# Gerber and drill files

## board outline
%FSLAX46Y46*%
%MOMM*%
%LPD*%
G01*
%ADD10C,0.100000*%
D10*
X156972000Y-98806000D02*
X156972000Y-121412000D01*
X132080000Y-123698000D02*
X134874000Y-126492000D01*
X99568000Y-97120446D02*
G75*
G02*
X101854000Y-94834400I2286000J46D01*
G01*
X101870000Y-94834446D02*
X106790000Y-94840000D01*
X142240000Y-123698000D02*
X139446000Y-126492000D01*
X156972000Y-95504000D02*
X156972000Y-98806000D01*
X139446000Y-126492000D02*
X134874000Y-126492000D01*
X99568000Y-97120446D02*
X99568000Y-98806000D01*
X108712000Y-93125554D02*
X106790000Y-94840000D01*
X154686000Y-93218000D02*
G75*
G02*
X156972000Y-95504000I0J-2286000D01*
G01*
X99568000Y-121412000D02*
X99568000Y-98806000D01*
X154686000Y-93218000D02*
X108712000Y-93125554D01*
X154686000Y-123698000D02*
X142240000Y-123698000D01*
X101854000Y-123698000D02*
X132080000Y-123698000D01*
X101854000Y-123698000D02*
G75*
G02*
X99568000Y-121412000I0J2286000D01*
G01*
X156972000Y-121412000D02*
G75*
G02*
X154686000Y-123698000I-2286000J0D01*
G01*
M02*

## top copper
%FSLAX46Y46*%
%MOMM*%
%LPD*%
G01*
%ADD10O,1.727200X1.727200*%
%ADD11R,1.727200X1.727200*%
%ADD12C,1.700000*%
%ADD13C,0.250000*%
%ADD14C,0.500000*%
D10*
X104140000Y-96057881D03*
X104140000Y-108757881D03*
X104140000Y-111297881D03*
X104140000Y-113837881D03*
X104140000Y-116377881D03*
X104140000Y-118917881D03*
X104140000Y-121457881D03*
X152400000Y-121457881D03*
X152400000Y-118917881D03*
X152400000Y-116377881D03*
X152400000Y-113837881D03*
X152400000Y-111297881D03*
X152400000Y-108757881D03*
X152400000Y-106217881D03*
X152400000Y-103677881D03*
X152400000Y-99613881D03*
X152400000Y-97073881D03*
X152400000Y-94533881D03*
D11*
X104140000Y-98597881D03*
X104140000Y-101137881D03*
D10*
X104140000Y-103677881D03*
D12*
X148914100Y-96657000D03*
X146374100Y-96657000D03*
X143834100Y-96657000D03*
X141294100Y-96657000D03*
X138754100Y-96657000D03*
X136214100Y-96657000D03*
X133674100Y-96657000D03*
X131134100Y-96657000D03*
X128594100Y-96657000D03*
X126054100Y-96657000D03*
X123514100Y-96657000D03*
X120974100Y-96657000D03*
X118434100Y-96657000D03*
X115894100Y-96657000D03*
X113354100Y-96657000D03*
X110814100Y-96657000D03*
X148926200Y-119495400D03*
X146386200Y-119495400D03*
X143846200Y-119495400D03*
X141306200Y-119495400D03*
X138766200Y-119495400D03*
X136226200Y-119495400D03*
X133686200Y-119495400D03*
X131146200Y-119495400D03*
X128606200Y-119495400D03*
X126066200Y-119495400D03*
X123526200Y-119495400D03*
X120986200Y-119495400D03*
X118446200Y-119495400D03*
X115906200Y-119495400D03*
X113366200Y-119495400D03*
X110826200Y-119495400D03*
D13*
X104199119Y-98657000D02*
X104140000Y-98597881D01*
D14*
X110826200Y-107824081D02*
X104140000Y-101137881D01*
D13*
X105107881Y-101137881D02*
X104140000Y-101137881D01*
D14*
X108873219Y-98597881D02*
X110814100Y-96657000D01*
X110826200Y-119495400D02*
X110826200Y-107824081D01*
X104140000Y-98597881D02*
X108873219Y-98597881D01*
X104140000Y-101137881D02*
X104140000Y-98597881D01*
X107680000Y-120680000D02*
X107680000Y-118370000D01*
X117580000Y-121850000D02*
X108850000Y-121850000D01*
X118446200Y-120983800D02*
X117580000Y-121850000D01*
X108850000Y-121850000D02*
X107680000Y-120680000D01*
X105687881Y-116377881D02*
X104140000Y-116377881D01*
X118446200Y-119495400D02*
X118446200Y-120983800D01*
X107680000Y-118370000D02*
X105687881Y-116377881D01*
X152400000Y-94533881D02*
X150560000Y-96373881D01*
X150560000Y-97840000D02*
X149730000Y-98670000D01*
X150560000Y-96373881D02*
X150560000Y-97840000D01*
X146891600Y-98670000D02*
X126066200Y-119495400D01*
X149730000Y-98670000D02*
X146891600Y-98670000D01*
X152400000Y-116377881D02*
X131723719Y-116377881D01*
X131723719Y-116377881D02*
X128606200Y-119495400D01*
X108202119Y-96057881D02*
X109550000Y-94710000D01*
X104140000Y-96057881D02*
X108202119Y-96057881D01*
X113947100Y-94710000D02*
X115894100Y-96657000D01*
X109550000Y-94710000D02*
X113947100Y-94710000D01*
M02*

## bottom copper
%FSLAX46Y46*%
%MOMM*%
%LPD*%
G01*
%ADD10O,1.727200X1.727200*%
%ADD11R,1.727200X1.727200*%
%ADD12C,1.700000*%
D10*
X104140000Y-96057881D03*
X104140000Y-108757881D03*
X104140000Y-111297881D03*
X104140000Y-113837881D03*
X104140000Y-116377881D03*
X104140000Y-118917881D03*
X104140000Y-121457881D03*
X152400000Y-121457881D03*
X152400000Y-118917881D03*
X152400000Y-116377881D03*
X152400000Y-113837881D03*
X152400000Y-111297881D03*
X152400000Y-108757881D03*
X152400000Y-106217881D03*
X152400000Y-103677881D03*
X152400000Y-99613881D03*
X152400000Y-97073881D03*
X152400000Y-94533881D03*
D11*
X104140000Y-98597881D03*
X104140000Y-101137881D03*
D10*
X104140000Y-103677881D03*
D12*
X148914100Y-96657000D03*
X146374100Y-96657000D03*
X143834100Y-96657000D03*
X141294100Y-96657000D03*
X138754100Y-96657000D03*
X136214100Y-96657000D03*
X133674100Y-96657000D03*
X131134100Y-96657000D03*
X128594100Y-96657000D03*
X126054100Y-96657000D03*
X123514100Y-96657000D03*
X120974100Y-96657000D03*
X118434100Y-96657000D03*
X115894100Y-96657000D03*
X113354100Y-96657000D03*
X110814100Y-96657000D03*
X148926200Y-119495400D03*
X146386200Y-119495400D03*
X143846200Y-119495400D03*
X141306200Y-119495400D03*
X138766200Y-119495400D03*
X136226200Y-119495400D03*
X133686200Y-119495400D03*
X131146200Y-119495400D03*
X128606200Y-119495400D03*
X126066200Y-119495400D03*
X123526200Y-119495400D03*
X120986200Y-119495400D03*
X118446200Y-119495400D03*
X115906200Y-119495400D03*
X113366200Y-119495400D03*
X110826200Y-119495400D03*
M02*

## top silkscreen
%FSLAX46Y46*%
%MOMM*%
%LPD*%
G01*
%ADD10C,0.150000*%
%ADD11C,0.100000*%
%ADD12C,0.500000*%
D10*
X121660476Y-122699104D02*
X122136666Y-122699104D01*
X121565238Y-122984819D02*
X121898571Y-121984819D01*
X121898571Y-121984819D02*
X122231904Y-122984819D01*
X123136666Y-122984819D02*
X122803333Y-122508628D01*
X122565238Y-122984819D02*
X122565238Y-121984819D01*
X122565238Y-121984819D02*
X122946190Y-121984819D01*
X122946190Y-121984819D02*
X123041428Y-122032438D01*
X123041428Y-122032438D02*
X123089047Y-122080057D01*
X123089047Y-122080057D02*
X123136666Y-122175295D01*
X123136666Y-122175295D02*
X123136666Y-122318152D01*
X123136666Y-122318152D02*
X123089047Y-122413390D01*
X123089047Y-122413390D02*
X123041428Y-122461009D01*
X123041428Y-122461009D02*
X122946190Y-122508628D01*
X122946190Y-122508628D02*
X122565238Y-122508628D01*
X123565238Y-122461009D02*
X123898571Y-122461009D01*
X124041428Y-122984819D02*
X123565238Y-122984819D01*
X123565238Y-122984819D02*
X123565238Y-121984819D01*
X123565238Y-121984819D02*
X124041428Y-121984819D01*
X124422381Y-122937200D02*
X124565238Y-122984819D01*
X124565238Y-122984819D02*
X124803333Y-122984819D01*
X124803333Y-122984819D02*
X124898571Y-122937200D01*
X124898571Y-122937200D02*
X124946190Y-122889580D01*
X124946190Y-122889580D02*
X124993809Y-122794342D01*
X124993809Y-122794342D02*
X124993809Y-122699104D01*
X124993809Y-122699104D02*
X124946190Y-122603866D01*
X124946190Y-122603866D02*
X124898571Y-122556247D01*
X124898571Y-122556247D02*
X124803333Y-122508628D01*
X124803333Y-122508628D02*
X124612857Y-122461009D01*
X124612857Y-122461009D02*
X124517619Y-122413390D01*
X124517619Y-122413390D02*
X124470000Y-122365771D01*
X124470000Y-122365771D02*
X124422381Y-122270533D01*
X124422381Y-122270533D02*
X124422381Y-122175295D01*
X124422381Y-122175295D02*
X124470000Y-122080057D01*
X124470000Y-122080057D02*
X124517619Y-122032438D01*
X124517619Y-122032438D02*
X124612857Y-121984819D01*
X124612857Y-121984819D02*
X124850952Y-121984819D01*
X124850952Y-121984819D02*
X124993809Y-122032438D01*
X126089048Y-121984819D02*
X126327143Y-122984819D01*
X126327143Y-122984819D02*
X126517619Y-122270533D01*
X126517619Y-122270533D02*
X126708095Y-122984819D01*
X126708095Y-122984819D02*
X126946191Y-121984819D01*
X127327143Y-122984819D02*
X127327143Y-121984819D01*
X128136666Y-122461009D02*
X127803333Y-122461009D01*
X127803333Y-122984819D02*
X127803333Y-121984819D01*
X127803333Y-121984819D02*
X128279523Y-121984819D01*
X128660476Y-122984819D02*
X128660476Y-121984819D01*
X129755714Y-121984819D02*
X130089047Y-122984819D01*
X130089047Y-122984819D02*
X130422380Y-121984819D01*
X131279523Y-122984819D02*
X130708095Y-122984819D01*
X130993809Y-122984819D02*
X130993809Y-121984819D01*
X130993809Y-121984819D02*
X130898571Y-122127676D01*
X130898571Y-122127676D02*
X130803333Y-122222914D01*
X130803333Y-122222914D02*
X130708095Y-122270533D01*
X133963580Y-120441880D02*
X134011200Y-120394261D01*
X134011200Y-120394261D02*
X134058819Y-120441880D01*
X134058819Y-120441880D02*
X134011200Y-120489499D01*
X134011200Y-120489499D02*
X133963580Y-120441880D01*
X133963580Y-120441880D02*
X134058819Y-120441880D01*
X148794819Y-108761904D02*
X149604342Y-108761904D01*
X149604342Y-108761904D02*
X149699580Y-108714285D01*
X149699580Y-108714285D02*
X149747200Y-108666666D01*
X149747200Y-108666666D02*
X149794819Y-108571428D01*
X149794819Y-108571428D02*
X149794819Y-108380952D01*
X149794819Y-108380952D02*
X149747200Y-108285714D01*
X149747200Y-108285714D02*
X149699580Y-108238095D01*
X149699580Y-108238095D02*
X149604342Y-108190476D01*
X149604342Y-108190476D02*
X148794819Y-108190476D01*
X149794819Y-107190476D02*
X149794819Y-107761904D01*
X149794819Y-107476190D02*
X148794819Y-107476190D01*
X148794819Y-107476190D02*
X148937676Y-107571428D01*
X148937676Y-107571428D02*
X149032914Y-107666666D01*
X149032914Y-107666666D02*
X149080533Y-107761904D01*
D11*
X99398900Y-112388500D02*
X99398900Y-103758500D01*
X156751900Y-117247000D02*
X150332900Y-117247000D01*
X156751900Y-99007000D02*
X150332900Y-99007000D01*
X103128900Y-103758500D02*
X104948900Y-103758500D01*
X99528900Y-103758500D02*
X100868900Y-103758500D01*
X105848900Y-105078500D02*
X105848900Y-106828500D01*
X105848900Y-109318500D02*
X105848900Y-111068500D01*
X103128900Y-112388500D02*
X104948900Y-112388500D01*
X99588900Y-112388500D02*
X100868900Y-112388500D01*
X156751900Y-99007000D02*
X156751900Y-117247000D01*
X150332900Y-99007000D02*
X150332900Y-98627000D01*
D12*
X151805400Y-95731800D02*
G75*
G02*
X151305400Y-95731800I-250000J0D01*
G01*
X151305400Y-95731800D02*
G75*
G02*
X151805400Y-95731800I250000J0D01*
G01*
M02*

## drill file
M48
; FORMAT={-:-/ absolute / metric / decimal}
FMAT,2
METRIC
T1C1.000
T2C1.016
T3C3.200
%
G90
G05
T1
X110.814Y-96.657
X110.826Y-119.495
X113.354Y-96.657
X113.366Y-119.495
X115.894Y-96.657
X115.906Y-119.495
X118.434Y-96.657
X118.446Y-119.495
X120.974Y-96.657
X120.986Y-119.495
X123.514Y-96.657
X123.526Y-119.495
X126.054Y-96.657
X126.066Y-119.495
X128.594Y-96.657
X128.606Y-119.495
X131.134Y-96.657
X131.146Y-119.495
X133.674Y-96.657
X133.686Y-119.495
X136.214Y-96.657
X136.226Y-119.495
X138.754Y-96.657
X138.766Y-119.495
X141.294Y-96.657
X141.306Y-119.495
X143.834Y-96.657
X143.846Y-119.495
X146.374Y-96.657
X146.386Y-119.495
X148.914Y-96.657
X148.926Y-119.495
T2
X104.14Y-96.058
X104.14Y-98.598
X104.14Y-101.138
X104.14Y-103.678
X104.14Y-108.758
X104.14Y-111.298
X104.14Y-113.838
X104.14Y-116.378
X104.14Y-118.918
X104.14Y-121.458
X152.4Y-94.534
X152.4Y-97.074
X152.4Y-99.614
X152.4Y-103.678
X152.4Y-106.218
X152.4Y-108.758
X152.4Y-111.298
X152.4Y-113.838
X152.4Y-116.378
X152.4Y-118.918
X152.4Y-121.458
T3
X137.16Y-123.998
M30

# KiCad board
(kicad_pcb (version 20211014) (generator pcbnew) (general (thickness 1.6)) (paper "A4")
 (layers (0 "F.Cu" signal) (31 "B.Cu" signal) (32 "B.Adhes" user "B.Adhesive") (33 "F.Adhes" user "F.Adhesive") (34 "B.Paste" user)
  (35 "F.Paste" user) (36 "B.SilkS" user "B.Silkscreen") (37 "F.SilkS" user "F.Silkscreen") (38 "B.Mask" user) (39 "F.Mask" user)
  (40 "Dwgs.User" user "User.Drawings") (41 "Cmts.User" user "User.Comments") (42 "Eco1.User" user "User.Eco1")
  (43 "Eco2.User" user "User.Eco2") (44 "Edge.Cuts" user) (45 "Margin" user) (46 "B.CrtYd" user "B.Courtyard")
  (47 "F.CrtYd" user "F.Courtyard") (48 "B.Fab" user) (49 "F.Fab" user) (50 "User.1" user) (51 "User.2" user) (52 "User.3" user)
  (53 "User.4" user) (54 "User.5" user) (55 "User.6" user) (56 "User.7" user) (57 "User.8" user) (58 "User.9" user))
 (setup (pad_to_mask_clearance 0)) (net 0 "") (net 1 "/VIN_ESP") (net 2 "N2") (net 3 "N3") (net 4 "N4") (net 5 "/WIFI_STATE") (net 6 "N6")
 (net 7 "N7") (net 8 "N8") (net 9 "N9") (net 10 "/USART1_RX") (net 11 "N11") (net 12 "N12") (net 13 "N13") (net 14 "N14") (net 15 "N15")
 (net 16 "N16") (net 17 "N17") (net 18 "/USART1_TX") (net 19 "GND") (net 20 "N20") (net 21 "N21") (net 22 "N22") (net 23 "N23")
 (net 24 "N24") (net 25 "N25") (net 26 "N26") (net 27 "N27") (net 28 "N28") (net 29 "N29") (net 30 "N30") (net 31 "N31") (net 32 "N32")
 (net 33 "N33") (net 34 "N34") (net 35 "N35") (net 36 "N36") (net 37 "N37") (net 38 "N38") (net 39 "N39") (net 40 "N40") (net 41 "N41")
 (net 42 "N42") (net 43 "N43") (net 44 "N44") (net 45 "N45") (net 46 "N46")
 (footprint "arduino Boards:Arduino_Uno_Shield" (layer "F.Cu") (at 101.6 57.957881 -90)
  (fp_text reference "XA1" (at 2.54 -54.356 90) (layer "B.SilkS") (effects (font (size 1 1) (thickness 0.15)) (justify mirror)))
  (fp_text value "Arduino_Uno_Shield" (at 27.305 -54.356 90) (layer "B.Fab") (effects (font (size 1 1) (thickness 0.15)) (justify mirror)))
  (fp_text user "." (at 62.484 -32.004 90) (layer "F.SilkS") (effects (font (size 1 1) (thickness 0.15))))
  (pad "" np_thru_hole circle (at 66.04 -35.56 270) (size 3.2 3.2) (drill 3.2) (layers *.Cu *.Mask))
  (pad "5V1" thru_hole oval (at 38.1 -2.54 270) (size 1.7272 1.7272) (drill 1.016) (layers *.Cu *.Mask) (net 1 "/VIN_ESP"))
  (pad "A0" thru_hole oval (at 50.8 -2.54 270) (size 1.7272 1.7272) (drill 1.016) (layers *.Cu *.Mask) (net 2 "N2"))
  (pad "A1" thru_hole oval (at 53.34 -2.54 270) (size 1.7272 1.7272) (drill 1.016) (layers *.Cu *.Mask) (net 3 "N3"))
  (pad "A2" thru_hole oval (at 55.88 -2.54 270) (size 1.7272 1.7272) (drill 1.016) (layers *.Cu *.Mask) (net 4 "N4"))
  (pad "A3" thru_hole oval (at 58.42 -2.54 270) (size 1.7272 1.7272) (drill 1.016) (layers *.Cu *.Mask) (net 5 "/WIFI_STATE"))
  (pad "A4" thru_hole oval (at 60.96 -2.54 270) (size 1.7272 1.7272) (drill 1.016) (layers *.Cu *.Mask) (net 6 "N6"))
  (pad "A5" thru_hole oval (at 63.5 -2.54 270) (size 1.7272 1.7272) (drill 1.016) (layers *.Cu *.Mask) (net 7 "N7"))
  (pad "D0" thru_hole oval (at 63.5 -50.8 270) (size 1.7272 1.7272) (drill 1.016) (layers *.Cu *.Mask) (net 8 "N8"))
  (pad "D1" thru_hole oval (at 60.96 -50.8 270) (size 1.7272 1.7272) (drill 1.016) (layers *.Cu *.Mask) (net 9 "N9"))
  (pad "D2" thru_hole oval (at 58.42 -50.8 270) (size 1.7272 1.7272) (drill 1.016) (layers *.Cu *.Mask) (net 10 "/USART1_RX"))
  (pad "D3" thru_hole oval (at 55.88 -50.8 270) (size 1.7272 1.7272) (drill 1.016) (layers *.Cu *.Mask) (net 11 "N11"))
  (pad "D4" thru_hole oval (at 53.34 -50.8 270) (size 1.7272 1.7272) (drill 1.016) (layers *.Cu *.Mask) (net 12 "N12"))
  (pad "D5" thru_hole oval (at 50.8 -50.8 270) (size 1.7272 1.7272) (drill 1.016) (layers *.Cu *.Mask) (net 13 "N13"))
  (pad "D6" thru_hole oval (at 48.26 -50.8 270) (size 1.7272 1.7272) (drill 1.016) (layers *.Cu *.Mask) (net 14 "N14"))
  (pad "D7" thru_hole oval (at 45.72 -50.8 270) (size 1.7272 1.7272) (drill 1.016) (layers *.Cu *.Mask) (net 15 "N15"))
  (pad "D8" thru_hole oval (at 41.656 -50.8 270) (size 1.7272 1.7272) (drill 1.016) (layers *.Cu *.Mask) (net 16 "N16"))
  (pad "D9" thru_hole oval (at 39.116 -50.8 270) (size 1.7272 1.7272) (drill 1.016) (layers *.Cu *.Mask) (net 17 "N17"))
  (pad "D10" thru_hole oval (at 36.576 -50.8 270) (size 1.7272 1.7272) (drill 1.016) (layers *.Cu *.Mask) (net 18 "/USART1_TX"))
  (pad "GND2" thru_hole rect (at 40.64 -2.54 270) (size 1.7272 1.7272) (drill 1.016) (layers *.Cu *.Mask) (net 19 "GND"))
  (pad "GND3" thru_hole rect (at 43.18 -2.54 270) (size 1.7272 1.7272) (drill 1.016) (layers *.Cu *.Mask) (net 19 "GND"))
  (pad "VIN" thru_hole oval (at 45.72 -2.54 270) (size 1.7272 1.7272) (drill 1.016) (layers *.Cu *.Mask) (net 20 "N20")))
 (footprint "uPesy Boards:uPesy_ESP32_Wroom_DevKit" (layer "F.Cu") (at 129.94 108 -90)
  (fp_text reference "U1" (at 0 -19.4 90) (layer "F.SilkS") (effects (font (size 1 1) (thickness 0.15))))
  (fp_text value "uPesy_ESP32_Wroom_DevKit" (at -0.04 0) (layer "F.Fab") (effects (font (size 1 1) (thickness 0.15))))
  (fp_line (start 4.3885 30.5411) (end -4.2415 30.5411) (layer "F.SilkS") (width 0.1))
  (fp_line (start 9.247 -26.8119) (end 9.247 -20.3929) (layer "F.SilkS") (width 0.1))
  (fp_line (start -8.993 -26.8119) (end -8.993 -20.3929) (layer "F.SilkS") (width 0.1))
  (fp_line (start -4.2415 26.8111) (end -4.2415 24.9911) (layer "F.SilkS") (width 0.1))
  (fp_line (start -4.2415 30.4111) (end -4.2415 29.0711) (layer "F.SilkS") (width 0.1))
  (fp_line (start -2.9215 24.0911) (end -1.1715 24.0911) (layer "F.SilkS") (width 0.1))
  (fp_line (start 1.3185 24.0911) (end 3.0685 24.0911) (layer "F.SilkS") (width 0.1))
  (fp_line (start 4.3885 26.8111) (end 4.3885 24.9911) (layer "F.SilkS") (width 0.1))
  (fp_line (start 4.3885 30.3511) (end 4.3885 29.0711) (layer "F.SilkS") (width 0.1))
  (fp_line (start -8.993 -26.8119) (end 9.247 -26.8119) (layer "F.SilkS") (width 0.1))
  (fp_line (start -8.993 -20.3929) (end -9.373 -20.3929) (layer "F.SilkS") (width 0.1))
  (fp_circle (center -12.2682 -21.6154) (end -12.0182 -21.6154) (layer "F.SilkS") (width 0.5) (fill none))
  (pad "1" thru_hole circle (at -11.343 -18.9741 180) (size 1.7 1.7) (drill 1) (layers *.Cu *.Mask) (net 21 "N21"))
  (pad "2" thru_hole circle (at -11.343 -16.4341 180) (size 1.7 1.7) (drill 1) (layers *.Cu *.Mask) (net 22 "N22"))
  (pad "3" thru_hole circle (at -11.343 -13.8941 180) (size 1.7 1.7) (drill 1) (layers *.Cu *.Mask) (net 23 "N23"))
  (pad "4" thru_hole circle (at -11.343 -11.3541 180) (size 1.7 1.7) (drill 1) (layers *.Cu *.Mask) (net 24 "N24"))
  (pad "5" thru_hole circle (at -11.343 -8.8141 180) (size 1.7 1.7) (drill 1) (layers *.Cu *.Mask) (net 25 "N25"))
  (pad "6" thru_hole circle (at -11.343 -6.2741 180) (size 1.7 1.7) (drill 1) (layers *.Cu *.Mask) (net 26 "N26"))
  (pad "7" thru_hole circle (at -11.343 -3.7341 180) (size 1.7 1.7) (drill 1) (layers *.Cu *.Mask) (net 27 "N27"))
  (pad "8" thru_hole circle (at -11.343 -1.1941 180) (size 1.7 1.7) (drill 1) (layers *.Cu *.Mask) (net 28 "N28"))
  (pad "9" thru_hole circle (at -11.343 1.3459 180) (size 1.7 1.7) (drill 1) (layers *.Cu *.Mask) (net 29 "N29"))
  (pad "10" thru_hole circle (at -11.343 3.8859 180) (size 1.7 1.7) (drill 1) (layers *.Cu *.Mask) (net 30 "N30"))
  (pad "11" thru_hole circle (at -11.343 6.4259 180) (size 1.7 1.7) (drill 1) (layers *.Cu *.Mask) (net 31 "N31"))
  (pad "12" thru_hole circle (at -11.343 8.9659 180) (size 1.7 1.7) (drill 1) (layers *.Cu *.Mask) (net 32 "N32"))
  (pad "13" thru_hole circle (at -11.343 11.5059 180) (size 1.7 1.7) (drill 1) (layers *.Cu *.Mask) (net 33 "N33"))
  (pad "14" thru_hole circle (at -11.343 14.0459 180) (size 1.7 1.7) (drill 1) (layers *.Cu *.Mask) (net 1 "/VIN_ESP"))
  (pad "15" thru_hole circle (at -11.343 16.5859 180) (size 1.7 1.7) (drill 1) (layers *.Cu *.Mask) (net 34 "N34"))
  (pad "16" thru_hole circle (at -11.343 19.1259 180) (size 1.7 1.7) (drill 1) (layers *.Cu *.Mask) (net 19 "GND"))
  (pad "17" thru_hole circle (at 11.4954 -18.9862) (size 1.7 1.7) (drill 1) (layers *.Cu *.Mask) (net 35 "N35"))
  (pad "18" thru_hole circle (at 11.4954 -16.4462) (size 1.7 1.7) (drill 1) (layers *.Cu *.Mask) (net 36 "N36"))
  (pad "19" thru_hole circle (at 11.4954 -13.9062) (size 1.7 1.7) (drill 1) (layers *.Cu *.Mask) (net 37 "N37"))
  (pad "20" thru_hole circle (at 11.4954 -11.3662) (size 1.7 1.7) (drill 1) (layers *.Cu *.Mask) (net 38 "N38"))
  (pad "21" thru_hole circle (at 11.4954 -8.8262) (size 1.7 1.7) (drill 1) (layers *.Cu *.Mask) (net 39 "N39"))
  (pad "22" thru_hole circle (at 11.4954 -6.2862) (size 1.7 1.7) (drill 1) (layers *.Cu *.Mask) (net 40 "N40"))
  (pad "23" thru_hole circle (at 11.4954 -3.7462) (size 1.7 1.7) (drill 1) (layers *.Cu *.Mask) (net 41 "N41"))
  (pad "24" thru_hole circle (at 11.4954 -1.2062) (size 1.7 1.7) (drill 1) (layers *.Cu *.Mask) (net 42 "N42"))
  (pad "25" thru_hole circle (at 11.4954 1.3338) (size 1.7 1.7) (drill 1) (layers *.Cu *.Mask) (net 10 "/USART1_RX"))
  (pad "26" thru_hole circle (at 11.4954 3.8738) (size 1.7 1.7) (drill 1) (layers *.Cu *.Mask) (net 18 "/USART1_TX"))
  (pad "27" thru_hole circle (at 11.4954 6.4138) (size 1.7 1.7) (drill 1) (layers *.Cu *.Mask) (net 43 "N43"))
  (pad "28" thru_hole circle (at 11.4954 8.9538) (size 1.7 1.7) (drill 1) (layers *.Cu *.Mask) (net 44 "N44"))
  (pad "29" thru_hole circle (at 11.4954 11.4938) (size 1.7 1.7) (drill 1) (layers *.Cu *.Mask) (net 5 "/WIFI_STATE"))
  (pad "30" thru_hole circle (at 11.4954 14.0338) (size 1.7 1.7) (drill 1) (layers *.Cu *.Mask) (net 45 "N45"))
  (pad "31" thru_hole circle (at 11.4954 16.5738) (size 1.7 1.7) (drill 1) (layers *.Cu *.Mask) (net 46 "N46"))
  (pad "32" thru_hole circle (at 11.4954 19.1138) (size 1.7 1.7) (drill 1) (layers *.Cu *.Mask) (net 19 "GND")))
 (gr_line (start 156.972 98.806) (end 156.972 121.412) (layer "Edge.Cuts") (width 0.1))
 (gr_line (start 132.08 123.698) (end 134.874 126.492) (layer "Edge.Cuts") (width 0.1))
 (gr_arc (start 99.568 97.120446) (mid 100.237554 95.504) (end 101.854 94.834446) (layer "Edge.Cuts") (width 0.1))
 (gr_line (start 101.87 94.834446) (end 106.79 94.84) (layer "Edge.Cuts") (width 0.1))
 (gr_line (start 142.24 123.698) (end 139.446 126.492) (layer "Edge.Cuts") (width 0.1))
 (gr_line (start 156.972 95.504) (end 156.972 98.806) (layer "Edge.Cuts") (width 0.1))
 (gr_line (start 139.446 126.492) (end 134.874 126.492) (layer "Edge.Cuts") (width 0.1))
 (gr_line (start 99.568 97.120446) (end 99.568 98.806) (layer "Edge.Cuts") (width 0.1))
 (gr_line (start 108.712 93.125554) (end 106.79 94.84) (layer "Edge.Cuts") (width 0.1))
 (gr_arc (start 154.686 93.218) (mid 156.302446 93.887554) (end 156.972 95.504) (layer "Edge.Cuts") (width 0.1))
 (gr_line (start 99.568 121.412) (end 99.568 98.806) (layer "Edge.Cuts") (width 0.1))
 (gr_line (start 154.686 93.218) (end 108.712 93.125554) (layer "Edge.Cuts") (width 0.1))
 (gr_line (start 154.686 123.698) (end 142.24 123.698) (layer "Edge.Cuts") (width 0.1))
 (gr_line (start 101.854 123.698) (end 132.08 123.698) (layer "Edge.Cuts") (width 0.1))
 (gr_arc (start 101.854 123.698) (mid 100.237554 123.028446) (end 99.568 121.412) (layer "Edge.Cuts") (width 0.1))
 (gr_arc (start 156.972 121.412) (mid 156.302446 123.028446) (end 154.686 123.698) (layer "Edge.Cuts") (width 0.1))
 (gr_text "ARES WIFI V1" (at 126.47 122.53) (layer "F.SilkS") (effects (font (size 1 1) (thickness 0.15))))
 (segment (start 104.199119 98.657) (end 104.14 98.597881) (width 0.25) (layer "F.Cu") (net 19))
 (segment (start 110.8262 107.824081) (end 104.14 101.137881) (width 0.5) (layer "F.Cu") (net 19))
 (segment (start 105.107881 101.137881) (end 104.14 101.137881) (width 0.25) (layer "F.Cu") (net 19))
 (segment (start 108.873219 98.597881) (end 110.8141 96.657) (width 0.5) (layer "F.Cu") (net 19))
 (segment (start 110.8262 119.4954) (end 110.8262 107.824081) (width 0.5) (layer "F.Cu") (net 19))
 (segment (start 104.14 98.597881) (end 108.873219 98.597881) (width 0.5) (layer "F.Cu") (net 19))
 (segment (start 104.14 101.137881) (end 104.14 98.597881) (width 0.5) (layer "F.Cu") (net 19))
 (segment (start 107.68 120.68) (end 107.68 118.37) (width 0.5) (layer "F.Cu") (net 5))
 (segment (start 117.58 121.85) (end 108.85 121.85) (width 0.5) (layer "F.Cu") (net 5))
 (segment (start 118.4462 120.9838) (end 117.58 121.85) (width 0.5) (layer "F.Cu") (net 5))
 (segment (start 108.85 121.85) (end 107.68 120.68) (width 0.5) (layer "F.Cu") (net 5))
 (segment (start 105.687881 116.377881) (end 104.14 116.377881) (width 0.5) (layer "F.Cu") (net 5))
 (segment (start 118.4462 119.4954) (end 118.4462 120.9838) (width 0.5) (layer "F.Cu") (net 5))
 (segment (start 107.68 118.37) (end 105.687881 116.377881) (width 0.5) (layer "F.Cu") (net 5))
 (segment (start 152.4 94.533881) (end 150.56 96.373881) (width 0.5) (layer "F.Cu") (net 18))
 (segment (start 150.56 97.84) (end 149.73 98.67) (width 0.5) (layer "F.Cu") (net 18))
 (segment (start 150.56 96.373881) (end 150.56 97.84) (width 0.5) (layer "F.Cu") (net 18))
 (segment (start 146.8916 98.67) (end 126.0662 119.4954) (width 0.5) (layer "F.Cu") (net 18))
 (segment (start 149.73 98.67) (end 146.8916 98.67) (width 0.5) (layer "F.Cu") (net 18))
 (segment (start 152.4 116.377881) (end 131.723719 116.377881) (width 0.5) (layer "F.Cu") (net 10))
 (segment (start 131.723719 116.377881) (end 128.6062 119.4954) (width 0.5) (layer "F.Cu") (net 10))
 (segment (start 108.202119 96.057881) (end 109.55 94.71) (width 0.5) (layer "F.Cu") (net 1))
 (segment (start 104.14 96.057881) (end 108.202119 96.057881) (width 0.5) (layer "F.Cu") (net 1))
 (segment (start 113.9471 94.71) (end 115.8941 96.657) (width 0.5) (layer "F.Cu") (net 1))
 (segment (start 109.55 94.71) (end 113.9471 94.71) (width 0.5) (layer "F.Cu") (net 1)))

